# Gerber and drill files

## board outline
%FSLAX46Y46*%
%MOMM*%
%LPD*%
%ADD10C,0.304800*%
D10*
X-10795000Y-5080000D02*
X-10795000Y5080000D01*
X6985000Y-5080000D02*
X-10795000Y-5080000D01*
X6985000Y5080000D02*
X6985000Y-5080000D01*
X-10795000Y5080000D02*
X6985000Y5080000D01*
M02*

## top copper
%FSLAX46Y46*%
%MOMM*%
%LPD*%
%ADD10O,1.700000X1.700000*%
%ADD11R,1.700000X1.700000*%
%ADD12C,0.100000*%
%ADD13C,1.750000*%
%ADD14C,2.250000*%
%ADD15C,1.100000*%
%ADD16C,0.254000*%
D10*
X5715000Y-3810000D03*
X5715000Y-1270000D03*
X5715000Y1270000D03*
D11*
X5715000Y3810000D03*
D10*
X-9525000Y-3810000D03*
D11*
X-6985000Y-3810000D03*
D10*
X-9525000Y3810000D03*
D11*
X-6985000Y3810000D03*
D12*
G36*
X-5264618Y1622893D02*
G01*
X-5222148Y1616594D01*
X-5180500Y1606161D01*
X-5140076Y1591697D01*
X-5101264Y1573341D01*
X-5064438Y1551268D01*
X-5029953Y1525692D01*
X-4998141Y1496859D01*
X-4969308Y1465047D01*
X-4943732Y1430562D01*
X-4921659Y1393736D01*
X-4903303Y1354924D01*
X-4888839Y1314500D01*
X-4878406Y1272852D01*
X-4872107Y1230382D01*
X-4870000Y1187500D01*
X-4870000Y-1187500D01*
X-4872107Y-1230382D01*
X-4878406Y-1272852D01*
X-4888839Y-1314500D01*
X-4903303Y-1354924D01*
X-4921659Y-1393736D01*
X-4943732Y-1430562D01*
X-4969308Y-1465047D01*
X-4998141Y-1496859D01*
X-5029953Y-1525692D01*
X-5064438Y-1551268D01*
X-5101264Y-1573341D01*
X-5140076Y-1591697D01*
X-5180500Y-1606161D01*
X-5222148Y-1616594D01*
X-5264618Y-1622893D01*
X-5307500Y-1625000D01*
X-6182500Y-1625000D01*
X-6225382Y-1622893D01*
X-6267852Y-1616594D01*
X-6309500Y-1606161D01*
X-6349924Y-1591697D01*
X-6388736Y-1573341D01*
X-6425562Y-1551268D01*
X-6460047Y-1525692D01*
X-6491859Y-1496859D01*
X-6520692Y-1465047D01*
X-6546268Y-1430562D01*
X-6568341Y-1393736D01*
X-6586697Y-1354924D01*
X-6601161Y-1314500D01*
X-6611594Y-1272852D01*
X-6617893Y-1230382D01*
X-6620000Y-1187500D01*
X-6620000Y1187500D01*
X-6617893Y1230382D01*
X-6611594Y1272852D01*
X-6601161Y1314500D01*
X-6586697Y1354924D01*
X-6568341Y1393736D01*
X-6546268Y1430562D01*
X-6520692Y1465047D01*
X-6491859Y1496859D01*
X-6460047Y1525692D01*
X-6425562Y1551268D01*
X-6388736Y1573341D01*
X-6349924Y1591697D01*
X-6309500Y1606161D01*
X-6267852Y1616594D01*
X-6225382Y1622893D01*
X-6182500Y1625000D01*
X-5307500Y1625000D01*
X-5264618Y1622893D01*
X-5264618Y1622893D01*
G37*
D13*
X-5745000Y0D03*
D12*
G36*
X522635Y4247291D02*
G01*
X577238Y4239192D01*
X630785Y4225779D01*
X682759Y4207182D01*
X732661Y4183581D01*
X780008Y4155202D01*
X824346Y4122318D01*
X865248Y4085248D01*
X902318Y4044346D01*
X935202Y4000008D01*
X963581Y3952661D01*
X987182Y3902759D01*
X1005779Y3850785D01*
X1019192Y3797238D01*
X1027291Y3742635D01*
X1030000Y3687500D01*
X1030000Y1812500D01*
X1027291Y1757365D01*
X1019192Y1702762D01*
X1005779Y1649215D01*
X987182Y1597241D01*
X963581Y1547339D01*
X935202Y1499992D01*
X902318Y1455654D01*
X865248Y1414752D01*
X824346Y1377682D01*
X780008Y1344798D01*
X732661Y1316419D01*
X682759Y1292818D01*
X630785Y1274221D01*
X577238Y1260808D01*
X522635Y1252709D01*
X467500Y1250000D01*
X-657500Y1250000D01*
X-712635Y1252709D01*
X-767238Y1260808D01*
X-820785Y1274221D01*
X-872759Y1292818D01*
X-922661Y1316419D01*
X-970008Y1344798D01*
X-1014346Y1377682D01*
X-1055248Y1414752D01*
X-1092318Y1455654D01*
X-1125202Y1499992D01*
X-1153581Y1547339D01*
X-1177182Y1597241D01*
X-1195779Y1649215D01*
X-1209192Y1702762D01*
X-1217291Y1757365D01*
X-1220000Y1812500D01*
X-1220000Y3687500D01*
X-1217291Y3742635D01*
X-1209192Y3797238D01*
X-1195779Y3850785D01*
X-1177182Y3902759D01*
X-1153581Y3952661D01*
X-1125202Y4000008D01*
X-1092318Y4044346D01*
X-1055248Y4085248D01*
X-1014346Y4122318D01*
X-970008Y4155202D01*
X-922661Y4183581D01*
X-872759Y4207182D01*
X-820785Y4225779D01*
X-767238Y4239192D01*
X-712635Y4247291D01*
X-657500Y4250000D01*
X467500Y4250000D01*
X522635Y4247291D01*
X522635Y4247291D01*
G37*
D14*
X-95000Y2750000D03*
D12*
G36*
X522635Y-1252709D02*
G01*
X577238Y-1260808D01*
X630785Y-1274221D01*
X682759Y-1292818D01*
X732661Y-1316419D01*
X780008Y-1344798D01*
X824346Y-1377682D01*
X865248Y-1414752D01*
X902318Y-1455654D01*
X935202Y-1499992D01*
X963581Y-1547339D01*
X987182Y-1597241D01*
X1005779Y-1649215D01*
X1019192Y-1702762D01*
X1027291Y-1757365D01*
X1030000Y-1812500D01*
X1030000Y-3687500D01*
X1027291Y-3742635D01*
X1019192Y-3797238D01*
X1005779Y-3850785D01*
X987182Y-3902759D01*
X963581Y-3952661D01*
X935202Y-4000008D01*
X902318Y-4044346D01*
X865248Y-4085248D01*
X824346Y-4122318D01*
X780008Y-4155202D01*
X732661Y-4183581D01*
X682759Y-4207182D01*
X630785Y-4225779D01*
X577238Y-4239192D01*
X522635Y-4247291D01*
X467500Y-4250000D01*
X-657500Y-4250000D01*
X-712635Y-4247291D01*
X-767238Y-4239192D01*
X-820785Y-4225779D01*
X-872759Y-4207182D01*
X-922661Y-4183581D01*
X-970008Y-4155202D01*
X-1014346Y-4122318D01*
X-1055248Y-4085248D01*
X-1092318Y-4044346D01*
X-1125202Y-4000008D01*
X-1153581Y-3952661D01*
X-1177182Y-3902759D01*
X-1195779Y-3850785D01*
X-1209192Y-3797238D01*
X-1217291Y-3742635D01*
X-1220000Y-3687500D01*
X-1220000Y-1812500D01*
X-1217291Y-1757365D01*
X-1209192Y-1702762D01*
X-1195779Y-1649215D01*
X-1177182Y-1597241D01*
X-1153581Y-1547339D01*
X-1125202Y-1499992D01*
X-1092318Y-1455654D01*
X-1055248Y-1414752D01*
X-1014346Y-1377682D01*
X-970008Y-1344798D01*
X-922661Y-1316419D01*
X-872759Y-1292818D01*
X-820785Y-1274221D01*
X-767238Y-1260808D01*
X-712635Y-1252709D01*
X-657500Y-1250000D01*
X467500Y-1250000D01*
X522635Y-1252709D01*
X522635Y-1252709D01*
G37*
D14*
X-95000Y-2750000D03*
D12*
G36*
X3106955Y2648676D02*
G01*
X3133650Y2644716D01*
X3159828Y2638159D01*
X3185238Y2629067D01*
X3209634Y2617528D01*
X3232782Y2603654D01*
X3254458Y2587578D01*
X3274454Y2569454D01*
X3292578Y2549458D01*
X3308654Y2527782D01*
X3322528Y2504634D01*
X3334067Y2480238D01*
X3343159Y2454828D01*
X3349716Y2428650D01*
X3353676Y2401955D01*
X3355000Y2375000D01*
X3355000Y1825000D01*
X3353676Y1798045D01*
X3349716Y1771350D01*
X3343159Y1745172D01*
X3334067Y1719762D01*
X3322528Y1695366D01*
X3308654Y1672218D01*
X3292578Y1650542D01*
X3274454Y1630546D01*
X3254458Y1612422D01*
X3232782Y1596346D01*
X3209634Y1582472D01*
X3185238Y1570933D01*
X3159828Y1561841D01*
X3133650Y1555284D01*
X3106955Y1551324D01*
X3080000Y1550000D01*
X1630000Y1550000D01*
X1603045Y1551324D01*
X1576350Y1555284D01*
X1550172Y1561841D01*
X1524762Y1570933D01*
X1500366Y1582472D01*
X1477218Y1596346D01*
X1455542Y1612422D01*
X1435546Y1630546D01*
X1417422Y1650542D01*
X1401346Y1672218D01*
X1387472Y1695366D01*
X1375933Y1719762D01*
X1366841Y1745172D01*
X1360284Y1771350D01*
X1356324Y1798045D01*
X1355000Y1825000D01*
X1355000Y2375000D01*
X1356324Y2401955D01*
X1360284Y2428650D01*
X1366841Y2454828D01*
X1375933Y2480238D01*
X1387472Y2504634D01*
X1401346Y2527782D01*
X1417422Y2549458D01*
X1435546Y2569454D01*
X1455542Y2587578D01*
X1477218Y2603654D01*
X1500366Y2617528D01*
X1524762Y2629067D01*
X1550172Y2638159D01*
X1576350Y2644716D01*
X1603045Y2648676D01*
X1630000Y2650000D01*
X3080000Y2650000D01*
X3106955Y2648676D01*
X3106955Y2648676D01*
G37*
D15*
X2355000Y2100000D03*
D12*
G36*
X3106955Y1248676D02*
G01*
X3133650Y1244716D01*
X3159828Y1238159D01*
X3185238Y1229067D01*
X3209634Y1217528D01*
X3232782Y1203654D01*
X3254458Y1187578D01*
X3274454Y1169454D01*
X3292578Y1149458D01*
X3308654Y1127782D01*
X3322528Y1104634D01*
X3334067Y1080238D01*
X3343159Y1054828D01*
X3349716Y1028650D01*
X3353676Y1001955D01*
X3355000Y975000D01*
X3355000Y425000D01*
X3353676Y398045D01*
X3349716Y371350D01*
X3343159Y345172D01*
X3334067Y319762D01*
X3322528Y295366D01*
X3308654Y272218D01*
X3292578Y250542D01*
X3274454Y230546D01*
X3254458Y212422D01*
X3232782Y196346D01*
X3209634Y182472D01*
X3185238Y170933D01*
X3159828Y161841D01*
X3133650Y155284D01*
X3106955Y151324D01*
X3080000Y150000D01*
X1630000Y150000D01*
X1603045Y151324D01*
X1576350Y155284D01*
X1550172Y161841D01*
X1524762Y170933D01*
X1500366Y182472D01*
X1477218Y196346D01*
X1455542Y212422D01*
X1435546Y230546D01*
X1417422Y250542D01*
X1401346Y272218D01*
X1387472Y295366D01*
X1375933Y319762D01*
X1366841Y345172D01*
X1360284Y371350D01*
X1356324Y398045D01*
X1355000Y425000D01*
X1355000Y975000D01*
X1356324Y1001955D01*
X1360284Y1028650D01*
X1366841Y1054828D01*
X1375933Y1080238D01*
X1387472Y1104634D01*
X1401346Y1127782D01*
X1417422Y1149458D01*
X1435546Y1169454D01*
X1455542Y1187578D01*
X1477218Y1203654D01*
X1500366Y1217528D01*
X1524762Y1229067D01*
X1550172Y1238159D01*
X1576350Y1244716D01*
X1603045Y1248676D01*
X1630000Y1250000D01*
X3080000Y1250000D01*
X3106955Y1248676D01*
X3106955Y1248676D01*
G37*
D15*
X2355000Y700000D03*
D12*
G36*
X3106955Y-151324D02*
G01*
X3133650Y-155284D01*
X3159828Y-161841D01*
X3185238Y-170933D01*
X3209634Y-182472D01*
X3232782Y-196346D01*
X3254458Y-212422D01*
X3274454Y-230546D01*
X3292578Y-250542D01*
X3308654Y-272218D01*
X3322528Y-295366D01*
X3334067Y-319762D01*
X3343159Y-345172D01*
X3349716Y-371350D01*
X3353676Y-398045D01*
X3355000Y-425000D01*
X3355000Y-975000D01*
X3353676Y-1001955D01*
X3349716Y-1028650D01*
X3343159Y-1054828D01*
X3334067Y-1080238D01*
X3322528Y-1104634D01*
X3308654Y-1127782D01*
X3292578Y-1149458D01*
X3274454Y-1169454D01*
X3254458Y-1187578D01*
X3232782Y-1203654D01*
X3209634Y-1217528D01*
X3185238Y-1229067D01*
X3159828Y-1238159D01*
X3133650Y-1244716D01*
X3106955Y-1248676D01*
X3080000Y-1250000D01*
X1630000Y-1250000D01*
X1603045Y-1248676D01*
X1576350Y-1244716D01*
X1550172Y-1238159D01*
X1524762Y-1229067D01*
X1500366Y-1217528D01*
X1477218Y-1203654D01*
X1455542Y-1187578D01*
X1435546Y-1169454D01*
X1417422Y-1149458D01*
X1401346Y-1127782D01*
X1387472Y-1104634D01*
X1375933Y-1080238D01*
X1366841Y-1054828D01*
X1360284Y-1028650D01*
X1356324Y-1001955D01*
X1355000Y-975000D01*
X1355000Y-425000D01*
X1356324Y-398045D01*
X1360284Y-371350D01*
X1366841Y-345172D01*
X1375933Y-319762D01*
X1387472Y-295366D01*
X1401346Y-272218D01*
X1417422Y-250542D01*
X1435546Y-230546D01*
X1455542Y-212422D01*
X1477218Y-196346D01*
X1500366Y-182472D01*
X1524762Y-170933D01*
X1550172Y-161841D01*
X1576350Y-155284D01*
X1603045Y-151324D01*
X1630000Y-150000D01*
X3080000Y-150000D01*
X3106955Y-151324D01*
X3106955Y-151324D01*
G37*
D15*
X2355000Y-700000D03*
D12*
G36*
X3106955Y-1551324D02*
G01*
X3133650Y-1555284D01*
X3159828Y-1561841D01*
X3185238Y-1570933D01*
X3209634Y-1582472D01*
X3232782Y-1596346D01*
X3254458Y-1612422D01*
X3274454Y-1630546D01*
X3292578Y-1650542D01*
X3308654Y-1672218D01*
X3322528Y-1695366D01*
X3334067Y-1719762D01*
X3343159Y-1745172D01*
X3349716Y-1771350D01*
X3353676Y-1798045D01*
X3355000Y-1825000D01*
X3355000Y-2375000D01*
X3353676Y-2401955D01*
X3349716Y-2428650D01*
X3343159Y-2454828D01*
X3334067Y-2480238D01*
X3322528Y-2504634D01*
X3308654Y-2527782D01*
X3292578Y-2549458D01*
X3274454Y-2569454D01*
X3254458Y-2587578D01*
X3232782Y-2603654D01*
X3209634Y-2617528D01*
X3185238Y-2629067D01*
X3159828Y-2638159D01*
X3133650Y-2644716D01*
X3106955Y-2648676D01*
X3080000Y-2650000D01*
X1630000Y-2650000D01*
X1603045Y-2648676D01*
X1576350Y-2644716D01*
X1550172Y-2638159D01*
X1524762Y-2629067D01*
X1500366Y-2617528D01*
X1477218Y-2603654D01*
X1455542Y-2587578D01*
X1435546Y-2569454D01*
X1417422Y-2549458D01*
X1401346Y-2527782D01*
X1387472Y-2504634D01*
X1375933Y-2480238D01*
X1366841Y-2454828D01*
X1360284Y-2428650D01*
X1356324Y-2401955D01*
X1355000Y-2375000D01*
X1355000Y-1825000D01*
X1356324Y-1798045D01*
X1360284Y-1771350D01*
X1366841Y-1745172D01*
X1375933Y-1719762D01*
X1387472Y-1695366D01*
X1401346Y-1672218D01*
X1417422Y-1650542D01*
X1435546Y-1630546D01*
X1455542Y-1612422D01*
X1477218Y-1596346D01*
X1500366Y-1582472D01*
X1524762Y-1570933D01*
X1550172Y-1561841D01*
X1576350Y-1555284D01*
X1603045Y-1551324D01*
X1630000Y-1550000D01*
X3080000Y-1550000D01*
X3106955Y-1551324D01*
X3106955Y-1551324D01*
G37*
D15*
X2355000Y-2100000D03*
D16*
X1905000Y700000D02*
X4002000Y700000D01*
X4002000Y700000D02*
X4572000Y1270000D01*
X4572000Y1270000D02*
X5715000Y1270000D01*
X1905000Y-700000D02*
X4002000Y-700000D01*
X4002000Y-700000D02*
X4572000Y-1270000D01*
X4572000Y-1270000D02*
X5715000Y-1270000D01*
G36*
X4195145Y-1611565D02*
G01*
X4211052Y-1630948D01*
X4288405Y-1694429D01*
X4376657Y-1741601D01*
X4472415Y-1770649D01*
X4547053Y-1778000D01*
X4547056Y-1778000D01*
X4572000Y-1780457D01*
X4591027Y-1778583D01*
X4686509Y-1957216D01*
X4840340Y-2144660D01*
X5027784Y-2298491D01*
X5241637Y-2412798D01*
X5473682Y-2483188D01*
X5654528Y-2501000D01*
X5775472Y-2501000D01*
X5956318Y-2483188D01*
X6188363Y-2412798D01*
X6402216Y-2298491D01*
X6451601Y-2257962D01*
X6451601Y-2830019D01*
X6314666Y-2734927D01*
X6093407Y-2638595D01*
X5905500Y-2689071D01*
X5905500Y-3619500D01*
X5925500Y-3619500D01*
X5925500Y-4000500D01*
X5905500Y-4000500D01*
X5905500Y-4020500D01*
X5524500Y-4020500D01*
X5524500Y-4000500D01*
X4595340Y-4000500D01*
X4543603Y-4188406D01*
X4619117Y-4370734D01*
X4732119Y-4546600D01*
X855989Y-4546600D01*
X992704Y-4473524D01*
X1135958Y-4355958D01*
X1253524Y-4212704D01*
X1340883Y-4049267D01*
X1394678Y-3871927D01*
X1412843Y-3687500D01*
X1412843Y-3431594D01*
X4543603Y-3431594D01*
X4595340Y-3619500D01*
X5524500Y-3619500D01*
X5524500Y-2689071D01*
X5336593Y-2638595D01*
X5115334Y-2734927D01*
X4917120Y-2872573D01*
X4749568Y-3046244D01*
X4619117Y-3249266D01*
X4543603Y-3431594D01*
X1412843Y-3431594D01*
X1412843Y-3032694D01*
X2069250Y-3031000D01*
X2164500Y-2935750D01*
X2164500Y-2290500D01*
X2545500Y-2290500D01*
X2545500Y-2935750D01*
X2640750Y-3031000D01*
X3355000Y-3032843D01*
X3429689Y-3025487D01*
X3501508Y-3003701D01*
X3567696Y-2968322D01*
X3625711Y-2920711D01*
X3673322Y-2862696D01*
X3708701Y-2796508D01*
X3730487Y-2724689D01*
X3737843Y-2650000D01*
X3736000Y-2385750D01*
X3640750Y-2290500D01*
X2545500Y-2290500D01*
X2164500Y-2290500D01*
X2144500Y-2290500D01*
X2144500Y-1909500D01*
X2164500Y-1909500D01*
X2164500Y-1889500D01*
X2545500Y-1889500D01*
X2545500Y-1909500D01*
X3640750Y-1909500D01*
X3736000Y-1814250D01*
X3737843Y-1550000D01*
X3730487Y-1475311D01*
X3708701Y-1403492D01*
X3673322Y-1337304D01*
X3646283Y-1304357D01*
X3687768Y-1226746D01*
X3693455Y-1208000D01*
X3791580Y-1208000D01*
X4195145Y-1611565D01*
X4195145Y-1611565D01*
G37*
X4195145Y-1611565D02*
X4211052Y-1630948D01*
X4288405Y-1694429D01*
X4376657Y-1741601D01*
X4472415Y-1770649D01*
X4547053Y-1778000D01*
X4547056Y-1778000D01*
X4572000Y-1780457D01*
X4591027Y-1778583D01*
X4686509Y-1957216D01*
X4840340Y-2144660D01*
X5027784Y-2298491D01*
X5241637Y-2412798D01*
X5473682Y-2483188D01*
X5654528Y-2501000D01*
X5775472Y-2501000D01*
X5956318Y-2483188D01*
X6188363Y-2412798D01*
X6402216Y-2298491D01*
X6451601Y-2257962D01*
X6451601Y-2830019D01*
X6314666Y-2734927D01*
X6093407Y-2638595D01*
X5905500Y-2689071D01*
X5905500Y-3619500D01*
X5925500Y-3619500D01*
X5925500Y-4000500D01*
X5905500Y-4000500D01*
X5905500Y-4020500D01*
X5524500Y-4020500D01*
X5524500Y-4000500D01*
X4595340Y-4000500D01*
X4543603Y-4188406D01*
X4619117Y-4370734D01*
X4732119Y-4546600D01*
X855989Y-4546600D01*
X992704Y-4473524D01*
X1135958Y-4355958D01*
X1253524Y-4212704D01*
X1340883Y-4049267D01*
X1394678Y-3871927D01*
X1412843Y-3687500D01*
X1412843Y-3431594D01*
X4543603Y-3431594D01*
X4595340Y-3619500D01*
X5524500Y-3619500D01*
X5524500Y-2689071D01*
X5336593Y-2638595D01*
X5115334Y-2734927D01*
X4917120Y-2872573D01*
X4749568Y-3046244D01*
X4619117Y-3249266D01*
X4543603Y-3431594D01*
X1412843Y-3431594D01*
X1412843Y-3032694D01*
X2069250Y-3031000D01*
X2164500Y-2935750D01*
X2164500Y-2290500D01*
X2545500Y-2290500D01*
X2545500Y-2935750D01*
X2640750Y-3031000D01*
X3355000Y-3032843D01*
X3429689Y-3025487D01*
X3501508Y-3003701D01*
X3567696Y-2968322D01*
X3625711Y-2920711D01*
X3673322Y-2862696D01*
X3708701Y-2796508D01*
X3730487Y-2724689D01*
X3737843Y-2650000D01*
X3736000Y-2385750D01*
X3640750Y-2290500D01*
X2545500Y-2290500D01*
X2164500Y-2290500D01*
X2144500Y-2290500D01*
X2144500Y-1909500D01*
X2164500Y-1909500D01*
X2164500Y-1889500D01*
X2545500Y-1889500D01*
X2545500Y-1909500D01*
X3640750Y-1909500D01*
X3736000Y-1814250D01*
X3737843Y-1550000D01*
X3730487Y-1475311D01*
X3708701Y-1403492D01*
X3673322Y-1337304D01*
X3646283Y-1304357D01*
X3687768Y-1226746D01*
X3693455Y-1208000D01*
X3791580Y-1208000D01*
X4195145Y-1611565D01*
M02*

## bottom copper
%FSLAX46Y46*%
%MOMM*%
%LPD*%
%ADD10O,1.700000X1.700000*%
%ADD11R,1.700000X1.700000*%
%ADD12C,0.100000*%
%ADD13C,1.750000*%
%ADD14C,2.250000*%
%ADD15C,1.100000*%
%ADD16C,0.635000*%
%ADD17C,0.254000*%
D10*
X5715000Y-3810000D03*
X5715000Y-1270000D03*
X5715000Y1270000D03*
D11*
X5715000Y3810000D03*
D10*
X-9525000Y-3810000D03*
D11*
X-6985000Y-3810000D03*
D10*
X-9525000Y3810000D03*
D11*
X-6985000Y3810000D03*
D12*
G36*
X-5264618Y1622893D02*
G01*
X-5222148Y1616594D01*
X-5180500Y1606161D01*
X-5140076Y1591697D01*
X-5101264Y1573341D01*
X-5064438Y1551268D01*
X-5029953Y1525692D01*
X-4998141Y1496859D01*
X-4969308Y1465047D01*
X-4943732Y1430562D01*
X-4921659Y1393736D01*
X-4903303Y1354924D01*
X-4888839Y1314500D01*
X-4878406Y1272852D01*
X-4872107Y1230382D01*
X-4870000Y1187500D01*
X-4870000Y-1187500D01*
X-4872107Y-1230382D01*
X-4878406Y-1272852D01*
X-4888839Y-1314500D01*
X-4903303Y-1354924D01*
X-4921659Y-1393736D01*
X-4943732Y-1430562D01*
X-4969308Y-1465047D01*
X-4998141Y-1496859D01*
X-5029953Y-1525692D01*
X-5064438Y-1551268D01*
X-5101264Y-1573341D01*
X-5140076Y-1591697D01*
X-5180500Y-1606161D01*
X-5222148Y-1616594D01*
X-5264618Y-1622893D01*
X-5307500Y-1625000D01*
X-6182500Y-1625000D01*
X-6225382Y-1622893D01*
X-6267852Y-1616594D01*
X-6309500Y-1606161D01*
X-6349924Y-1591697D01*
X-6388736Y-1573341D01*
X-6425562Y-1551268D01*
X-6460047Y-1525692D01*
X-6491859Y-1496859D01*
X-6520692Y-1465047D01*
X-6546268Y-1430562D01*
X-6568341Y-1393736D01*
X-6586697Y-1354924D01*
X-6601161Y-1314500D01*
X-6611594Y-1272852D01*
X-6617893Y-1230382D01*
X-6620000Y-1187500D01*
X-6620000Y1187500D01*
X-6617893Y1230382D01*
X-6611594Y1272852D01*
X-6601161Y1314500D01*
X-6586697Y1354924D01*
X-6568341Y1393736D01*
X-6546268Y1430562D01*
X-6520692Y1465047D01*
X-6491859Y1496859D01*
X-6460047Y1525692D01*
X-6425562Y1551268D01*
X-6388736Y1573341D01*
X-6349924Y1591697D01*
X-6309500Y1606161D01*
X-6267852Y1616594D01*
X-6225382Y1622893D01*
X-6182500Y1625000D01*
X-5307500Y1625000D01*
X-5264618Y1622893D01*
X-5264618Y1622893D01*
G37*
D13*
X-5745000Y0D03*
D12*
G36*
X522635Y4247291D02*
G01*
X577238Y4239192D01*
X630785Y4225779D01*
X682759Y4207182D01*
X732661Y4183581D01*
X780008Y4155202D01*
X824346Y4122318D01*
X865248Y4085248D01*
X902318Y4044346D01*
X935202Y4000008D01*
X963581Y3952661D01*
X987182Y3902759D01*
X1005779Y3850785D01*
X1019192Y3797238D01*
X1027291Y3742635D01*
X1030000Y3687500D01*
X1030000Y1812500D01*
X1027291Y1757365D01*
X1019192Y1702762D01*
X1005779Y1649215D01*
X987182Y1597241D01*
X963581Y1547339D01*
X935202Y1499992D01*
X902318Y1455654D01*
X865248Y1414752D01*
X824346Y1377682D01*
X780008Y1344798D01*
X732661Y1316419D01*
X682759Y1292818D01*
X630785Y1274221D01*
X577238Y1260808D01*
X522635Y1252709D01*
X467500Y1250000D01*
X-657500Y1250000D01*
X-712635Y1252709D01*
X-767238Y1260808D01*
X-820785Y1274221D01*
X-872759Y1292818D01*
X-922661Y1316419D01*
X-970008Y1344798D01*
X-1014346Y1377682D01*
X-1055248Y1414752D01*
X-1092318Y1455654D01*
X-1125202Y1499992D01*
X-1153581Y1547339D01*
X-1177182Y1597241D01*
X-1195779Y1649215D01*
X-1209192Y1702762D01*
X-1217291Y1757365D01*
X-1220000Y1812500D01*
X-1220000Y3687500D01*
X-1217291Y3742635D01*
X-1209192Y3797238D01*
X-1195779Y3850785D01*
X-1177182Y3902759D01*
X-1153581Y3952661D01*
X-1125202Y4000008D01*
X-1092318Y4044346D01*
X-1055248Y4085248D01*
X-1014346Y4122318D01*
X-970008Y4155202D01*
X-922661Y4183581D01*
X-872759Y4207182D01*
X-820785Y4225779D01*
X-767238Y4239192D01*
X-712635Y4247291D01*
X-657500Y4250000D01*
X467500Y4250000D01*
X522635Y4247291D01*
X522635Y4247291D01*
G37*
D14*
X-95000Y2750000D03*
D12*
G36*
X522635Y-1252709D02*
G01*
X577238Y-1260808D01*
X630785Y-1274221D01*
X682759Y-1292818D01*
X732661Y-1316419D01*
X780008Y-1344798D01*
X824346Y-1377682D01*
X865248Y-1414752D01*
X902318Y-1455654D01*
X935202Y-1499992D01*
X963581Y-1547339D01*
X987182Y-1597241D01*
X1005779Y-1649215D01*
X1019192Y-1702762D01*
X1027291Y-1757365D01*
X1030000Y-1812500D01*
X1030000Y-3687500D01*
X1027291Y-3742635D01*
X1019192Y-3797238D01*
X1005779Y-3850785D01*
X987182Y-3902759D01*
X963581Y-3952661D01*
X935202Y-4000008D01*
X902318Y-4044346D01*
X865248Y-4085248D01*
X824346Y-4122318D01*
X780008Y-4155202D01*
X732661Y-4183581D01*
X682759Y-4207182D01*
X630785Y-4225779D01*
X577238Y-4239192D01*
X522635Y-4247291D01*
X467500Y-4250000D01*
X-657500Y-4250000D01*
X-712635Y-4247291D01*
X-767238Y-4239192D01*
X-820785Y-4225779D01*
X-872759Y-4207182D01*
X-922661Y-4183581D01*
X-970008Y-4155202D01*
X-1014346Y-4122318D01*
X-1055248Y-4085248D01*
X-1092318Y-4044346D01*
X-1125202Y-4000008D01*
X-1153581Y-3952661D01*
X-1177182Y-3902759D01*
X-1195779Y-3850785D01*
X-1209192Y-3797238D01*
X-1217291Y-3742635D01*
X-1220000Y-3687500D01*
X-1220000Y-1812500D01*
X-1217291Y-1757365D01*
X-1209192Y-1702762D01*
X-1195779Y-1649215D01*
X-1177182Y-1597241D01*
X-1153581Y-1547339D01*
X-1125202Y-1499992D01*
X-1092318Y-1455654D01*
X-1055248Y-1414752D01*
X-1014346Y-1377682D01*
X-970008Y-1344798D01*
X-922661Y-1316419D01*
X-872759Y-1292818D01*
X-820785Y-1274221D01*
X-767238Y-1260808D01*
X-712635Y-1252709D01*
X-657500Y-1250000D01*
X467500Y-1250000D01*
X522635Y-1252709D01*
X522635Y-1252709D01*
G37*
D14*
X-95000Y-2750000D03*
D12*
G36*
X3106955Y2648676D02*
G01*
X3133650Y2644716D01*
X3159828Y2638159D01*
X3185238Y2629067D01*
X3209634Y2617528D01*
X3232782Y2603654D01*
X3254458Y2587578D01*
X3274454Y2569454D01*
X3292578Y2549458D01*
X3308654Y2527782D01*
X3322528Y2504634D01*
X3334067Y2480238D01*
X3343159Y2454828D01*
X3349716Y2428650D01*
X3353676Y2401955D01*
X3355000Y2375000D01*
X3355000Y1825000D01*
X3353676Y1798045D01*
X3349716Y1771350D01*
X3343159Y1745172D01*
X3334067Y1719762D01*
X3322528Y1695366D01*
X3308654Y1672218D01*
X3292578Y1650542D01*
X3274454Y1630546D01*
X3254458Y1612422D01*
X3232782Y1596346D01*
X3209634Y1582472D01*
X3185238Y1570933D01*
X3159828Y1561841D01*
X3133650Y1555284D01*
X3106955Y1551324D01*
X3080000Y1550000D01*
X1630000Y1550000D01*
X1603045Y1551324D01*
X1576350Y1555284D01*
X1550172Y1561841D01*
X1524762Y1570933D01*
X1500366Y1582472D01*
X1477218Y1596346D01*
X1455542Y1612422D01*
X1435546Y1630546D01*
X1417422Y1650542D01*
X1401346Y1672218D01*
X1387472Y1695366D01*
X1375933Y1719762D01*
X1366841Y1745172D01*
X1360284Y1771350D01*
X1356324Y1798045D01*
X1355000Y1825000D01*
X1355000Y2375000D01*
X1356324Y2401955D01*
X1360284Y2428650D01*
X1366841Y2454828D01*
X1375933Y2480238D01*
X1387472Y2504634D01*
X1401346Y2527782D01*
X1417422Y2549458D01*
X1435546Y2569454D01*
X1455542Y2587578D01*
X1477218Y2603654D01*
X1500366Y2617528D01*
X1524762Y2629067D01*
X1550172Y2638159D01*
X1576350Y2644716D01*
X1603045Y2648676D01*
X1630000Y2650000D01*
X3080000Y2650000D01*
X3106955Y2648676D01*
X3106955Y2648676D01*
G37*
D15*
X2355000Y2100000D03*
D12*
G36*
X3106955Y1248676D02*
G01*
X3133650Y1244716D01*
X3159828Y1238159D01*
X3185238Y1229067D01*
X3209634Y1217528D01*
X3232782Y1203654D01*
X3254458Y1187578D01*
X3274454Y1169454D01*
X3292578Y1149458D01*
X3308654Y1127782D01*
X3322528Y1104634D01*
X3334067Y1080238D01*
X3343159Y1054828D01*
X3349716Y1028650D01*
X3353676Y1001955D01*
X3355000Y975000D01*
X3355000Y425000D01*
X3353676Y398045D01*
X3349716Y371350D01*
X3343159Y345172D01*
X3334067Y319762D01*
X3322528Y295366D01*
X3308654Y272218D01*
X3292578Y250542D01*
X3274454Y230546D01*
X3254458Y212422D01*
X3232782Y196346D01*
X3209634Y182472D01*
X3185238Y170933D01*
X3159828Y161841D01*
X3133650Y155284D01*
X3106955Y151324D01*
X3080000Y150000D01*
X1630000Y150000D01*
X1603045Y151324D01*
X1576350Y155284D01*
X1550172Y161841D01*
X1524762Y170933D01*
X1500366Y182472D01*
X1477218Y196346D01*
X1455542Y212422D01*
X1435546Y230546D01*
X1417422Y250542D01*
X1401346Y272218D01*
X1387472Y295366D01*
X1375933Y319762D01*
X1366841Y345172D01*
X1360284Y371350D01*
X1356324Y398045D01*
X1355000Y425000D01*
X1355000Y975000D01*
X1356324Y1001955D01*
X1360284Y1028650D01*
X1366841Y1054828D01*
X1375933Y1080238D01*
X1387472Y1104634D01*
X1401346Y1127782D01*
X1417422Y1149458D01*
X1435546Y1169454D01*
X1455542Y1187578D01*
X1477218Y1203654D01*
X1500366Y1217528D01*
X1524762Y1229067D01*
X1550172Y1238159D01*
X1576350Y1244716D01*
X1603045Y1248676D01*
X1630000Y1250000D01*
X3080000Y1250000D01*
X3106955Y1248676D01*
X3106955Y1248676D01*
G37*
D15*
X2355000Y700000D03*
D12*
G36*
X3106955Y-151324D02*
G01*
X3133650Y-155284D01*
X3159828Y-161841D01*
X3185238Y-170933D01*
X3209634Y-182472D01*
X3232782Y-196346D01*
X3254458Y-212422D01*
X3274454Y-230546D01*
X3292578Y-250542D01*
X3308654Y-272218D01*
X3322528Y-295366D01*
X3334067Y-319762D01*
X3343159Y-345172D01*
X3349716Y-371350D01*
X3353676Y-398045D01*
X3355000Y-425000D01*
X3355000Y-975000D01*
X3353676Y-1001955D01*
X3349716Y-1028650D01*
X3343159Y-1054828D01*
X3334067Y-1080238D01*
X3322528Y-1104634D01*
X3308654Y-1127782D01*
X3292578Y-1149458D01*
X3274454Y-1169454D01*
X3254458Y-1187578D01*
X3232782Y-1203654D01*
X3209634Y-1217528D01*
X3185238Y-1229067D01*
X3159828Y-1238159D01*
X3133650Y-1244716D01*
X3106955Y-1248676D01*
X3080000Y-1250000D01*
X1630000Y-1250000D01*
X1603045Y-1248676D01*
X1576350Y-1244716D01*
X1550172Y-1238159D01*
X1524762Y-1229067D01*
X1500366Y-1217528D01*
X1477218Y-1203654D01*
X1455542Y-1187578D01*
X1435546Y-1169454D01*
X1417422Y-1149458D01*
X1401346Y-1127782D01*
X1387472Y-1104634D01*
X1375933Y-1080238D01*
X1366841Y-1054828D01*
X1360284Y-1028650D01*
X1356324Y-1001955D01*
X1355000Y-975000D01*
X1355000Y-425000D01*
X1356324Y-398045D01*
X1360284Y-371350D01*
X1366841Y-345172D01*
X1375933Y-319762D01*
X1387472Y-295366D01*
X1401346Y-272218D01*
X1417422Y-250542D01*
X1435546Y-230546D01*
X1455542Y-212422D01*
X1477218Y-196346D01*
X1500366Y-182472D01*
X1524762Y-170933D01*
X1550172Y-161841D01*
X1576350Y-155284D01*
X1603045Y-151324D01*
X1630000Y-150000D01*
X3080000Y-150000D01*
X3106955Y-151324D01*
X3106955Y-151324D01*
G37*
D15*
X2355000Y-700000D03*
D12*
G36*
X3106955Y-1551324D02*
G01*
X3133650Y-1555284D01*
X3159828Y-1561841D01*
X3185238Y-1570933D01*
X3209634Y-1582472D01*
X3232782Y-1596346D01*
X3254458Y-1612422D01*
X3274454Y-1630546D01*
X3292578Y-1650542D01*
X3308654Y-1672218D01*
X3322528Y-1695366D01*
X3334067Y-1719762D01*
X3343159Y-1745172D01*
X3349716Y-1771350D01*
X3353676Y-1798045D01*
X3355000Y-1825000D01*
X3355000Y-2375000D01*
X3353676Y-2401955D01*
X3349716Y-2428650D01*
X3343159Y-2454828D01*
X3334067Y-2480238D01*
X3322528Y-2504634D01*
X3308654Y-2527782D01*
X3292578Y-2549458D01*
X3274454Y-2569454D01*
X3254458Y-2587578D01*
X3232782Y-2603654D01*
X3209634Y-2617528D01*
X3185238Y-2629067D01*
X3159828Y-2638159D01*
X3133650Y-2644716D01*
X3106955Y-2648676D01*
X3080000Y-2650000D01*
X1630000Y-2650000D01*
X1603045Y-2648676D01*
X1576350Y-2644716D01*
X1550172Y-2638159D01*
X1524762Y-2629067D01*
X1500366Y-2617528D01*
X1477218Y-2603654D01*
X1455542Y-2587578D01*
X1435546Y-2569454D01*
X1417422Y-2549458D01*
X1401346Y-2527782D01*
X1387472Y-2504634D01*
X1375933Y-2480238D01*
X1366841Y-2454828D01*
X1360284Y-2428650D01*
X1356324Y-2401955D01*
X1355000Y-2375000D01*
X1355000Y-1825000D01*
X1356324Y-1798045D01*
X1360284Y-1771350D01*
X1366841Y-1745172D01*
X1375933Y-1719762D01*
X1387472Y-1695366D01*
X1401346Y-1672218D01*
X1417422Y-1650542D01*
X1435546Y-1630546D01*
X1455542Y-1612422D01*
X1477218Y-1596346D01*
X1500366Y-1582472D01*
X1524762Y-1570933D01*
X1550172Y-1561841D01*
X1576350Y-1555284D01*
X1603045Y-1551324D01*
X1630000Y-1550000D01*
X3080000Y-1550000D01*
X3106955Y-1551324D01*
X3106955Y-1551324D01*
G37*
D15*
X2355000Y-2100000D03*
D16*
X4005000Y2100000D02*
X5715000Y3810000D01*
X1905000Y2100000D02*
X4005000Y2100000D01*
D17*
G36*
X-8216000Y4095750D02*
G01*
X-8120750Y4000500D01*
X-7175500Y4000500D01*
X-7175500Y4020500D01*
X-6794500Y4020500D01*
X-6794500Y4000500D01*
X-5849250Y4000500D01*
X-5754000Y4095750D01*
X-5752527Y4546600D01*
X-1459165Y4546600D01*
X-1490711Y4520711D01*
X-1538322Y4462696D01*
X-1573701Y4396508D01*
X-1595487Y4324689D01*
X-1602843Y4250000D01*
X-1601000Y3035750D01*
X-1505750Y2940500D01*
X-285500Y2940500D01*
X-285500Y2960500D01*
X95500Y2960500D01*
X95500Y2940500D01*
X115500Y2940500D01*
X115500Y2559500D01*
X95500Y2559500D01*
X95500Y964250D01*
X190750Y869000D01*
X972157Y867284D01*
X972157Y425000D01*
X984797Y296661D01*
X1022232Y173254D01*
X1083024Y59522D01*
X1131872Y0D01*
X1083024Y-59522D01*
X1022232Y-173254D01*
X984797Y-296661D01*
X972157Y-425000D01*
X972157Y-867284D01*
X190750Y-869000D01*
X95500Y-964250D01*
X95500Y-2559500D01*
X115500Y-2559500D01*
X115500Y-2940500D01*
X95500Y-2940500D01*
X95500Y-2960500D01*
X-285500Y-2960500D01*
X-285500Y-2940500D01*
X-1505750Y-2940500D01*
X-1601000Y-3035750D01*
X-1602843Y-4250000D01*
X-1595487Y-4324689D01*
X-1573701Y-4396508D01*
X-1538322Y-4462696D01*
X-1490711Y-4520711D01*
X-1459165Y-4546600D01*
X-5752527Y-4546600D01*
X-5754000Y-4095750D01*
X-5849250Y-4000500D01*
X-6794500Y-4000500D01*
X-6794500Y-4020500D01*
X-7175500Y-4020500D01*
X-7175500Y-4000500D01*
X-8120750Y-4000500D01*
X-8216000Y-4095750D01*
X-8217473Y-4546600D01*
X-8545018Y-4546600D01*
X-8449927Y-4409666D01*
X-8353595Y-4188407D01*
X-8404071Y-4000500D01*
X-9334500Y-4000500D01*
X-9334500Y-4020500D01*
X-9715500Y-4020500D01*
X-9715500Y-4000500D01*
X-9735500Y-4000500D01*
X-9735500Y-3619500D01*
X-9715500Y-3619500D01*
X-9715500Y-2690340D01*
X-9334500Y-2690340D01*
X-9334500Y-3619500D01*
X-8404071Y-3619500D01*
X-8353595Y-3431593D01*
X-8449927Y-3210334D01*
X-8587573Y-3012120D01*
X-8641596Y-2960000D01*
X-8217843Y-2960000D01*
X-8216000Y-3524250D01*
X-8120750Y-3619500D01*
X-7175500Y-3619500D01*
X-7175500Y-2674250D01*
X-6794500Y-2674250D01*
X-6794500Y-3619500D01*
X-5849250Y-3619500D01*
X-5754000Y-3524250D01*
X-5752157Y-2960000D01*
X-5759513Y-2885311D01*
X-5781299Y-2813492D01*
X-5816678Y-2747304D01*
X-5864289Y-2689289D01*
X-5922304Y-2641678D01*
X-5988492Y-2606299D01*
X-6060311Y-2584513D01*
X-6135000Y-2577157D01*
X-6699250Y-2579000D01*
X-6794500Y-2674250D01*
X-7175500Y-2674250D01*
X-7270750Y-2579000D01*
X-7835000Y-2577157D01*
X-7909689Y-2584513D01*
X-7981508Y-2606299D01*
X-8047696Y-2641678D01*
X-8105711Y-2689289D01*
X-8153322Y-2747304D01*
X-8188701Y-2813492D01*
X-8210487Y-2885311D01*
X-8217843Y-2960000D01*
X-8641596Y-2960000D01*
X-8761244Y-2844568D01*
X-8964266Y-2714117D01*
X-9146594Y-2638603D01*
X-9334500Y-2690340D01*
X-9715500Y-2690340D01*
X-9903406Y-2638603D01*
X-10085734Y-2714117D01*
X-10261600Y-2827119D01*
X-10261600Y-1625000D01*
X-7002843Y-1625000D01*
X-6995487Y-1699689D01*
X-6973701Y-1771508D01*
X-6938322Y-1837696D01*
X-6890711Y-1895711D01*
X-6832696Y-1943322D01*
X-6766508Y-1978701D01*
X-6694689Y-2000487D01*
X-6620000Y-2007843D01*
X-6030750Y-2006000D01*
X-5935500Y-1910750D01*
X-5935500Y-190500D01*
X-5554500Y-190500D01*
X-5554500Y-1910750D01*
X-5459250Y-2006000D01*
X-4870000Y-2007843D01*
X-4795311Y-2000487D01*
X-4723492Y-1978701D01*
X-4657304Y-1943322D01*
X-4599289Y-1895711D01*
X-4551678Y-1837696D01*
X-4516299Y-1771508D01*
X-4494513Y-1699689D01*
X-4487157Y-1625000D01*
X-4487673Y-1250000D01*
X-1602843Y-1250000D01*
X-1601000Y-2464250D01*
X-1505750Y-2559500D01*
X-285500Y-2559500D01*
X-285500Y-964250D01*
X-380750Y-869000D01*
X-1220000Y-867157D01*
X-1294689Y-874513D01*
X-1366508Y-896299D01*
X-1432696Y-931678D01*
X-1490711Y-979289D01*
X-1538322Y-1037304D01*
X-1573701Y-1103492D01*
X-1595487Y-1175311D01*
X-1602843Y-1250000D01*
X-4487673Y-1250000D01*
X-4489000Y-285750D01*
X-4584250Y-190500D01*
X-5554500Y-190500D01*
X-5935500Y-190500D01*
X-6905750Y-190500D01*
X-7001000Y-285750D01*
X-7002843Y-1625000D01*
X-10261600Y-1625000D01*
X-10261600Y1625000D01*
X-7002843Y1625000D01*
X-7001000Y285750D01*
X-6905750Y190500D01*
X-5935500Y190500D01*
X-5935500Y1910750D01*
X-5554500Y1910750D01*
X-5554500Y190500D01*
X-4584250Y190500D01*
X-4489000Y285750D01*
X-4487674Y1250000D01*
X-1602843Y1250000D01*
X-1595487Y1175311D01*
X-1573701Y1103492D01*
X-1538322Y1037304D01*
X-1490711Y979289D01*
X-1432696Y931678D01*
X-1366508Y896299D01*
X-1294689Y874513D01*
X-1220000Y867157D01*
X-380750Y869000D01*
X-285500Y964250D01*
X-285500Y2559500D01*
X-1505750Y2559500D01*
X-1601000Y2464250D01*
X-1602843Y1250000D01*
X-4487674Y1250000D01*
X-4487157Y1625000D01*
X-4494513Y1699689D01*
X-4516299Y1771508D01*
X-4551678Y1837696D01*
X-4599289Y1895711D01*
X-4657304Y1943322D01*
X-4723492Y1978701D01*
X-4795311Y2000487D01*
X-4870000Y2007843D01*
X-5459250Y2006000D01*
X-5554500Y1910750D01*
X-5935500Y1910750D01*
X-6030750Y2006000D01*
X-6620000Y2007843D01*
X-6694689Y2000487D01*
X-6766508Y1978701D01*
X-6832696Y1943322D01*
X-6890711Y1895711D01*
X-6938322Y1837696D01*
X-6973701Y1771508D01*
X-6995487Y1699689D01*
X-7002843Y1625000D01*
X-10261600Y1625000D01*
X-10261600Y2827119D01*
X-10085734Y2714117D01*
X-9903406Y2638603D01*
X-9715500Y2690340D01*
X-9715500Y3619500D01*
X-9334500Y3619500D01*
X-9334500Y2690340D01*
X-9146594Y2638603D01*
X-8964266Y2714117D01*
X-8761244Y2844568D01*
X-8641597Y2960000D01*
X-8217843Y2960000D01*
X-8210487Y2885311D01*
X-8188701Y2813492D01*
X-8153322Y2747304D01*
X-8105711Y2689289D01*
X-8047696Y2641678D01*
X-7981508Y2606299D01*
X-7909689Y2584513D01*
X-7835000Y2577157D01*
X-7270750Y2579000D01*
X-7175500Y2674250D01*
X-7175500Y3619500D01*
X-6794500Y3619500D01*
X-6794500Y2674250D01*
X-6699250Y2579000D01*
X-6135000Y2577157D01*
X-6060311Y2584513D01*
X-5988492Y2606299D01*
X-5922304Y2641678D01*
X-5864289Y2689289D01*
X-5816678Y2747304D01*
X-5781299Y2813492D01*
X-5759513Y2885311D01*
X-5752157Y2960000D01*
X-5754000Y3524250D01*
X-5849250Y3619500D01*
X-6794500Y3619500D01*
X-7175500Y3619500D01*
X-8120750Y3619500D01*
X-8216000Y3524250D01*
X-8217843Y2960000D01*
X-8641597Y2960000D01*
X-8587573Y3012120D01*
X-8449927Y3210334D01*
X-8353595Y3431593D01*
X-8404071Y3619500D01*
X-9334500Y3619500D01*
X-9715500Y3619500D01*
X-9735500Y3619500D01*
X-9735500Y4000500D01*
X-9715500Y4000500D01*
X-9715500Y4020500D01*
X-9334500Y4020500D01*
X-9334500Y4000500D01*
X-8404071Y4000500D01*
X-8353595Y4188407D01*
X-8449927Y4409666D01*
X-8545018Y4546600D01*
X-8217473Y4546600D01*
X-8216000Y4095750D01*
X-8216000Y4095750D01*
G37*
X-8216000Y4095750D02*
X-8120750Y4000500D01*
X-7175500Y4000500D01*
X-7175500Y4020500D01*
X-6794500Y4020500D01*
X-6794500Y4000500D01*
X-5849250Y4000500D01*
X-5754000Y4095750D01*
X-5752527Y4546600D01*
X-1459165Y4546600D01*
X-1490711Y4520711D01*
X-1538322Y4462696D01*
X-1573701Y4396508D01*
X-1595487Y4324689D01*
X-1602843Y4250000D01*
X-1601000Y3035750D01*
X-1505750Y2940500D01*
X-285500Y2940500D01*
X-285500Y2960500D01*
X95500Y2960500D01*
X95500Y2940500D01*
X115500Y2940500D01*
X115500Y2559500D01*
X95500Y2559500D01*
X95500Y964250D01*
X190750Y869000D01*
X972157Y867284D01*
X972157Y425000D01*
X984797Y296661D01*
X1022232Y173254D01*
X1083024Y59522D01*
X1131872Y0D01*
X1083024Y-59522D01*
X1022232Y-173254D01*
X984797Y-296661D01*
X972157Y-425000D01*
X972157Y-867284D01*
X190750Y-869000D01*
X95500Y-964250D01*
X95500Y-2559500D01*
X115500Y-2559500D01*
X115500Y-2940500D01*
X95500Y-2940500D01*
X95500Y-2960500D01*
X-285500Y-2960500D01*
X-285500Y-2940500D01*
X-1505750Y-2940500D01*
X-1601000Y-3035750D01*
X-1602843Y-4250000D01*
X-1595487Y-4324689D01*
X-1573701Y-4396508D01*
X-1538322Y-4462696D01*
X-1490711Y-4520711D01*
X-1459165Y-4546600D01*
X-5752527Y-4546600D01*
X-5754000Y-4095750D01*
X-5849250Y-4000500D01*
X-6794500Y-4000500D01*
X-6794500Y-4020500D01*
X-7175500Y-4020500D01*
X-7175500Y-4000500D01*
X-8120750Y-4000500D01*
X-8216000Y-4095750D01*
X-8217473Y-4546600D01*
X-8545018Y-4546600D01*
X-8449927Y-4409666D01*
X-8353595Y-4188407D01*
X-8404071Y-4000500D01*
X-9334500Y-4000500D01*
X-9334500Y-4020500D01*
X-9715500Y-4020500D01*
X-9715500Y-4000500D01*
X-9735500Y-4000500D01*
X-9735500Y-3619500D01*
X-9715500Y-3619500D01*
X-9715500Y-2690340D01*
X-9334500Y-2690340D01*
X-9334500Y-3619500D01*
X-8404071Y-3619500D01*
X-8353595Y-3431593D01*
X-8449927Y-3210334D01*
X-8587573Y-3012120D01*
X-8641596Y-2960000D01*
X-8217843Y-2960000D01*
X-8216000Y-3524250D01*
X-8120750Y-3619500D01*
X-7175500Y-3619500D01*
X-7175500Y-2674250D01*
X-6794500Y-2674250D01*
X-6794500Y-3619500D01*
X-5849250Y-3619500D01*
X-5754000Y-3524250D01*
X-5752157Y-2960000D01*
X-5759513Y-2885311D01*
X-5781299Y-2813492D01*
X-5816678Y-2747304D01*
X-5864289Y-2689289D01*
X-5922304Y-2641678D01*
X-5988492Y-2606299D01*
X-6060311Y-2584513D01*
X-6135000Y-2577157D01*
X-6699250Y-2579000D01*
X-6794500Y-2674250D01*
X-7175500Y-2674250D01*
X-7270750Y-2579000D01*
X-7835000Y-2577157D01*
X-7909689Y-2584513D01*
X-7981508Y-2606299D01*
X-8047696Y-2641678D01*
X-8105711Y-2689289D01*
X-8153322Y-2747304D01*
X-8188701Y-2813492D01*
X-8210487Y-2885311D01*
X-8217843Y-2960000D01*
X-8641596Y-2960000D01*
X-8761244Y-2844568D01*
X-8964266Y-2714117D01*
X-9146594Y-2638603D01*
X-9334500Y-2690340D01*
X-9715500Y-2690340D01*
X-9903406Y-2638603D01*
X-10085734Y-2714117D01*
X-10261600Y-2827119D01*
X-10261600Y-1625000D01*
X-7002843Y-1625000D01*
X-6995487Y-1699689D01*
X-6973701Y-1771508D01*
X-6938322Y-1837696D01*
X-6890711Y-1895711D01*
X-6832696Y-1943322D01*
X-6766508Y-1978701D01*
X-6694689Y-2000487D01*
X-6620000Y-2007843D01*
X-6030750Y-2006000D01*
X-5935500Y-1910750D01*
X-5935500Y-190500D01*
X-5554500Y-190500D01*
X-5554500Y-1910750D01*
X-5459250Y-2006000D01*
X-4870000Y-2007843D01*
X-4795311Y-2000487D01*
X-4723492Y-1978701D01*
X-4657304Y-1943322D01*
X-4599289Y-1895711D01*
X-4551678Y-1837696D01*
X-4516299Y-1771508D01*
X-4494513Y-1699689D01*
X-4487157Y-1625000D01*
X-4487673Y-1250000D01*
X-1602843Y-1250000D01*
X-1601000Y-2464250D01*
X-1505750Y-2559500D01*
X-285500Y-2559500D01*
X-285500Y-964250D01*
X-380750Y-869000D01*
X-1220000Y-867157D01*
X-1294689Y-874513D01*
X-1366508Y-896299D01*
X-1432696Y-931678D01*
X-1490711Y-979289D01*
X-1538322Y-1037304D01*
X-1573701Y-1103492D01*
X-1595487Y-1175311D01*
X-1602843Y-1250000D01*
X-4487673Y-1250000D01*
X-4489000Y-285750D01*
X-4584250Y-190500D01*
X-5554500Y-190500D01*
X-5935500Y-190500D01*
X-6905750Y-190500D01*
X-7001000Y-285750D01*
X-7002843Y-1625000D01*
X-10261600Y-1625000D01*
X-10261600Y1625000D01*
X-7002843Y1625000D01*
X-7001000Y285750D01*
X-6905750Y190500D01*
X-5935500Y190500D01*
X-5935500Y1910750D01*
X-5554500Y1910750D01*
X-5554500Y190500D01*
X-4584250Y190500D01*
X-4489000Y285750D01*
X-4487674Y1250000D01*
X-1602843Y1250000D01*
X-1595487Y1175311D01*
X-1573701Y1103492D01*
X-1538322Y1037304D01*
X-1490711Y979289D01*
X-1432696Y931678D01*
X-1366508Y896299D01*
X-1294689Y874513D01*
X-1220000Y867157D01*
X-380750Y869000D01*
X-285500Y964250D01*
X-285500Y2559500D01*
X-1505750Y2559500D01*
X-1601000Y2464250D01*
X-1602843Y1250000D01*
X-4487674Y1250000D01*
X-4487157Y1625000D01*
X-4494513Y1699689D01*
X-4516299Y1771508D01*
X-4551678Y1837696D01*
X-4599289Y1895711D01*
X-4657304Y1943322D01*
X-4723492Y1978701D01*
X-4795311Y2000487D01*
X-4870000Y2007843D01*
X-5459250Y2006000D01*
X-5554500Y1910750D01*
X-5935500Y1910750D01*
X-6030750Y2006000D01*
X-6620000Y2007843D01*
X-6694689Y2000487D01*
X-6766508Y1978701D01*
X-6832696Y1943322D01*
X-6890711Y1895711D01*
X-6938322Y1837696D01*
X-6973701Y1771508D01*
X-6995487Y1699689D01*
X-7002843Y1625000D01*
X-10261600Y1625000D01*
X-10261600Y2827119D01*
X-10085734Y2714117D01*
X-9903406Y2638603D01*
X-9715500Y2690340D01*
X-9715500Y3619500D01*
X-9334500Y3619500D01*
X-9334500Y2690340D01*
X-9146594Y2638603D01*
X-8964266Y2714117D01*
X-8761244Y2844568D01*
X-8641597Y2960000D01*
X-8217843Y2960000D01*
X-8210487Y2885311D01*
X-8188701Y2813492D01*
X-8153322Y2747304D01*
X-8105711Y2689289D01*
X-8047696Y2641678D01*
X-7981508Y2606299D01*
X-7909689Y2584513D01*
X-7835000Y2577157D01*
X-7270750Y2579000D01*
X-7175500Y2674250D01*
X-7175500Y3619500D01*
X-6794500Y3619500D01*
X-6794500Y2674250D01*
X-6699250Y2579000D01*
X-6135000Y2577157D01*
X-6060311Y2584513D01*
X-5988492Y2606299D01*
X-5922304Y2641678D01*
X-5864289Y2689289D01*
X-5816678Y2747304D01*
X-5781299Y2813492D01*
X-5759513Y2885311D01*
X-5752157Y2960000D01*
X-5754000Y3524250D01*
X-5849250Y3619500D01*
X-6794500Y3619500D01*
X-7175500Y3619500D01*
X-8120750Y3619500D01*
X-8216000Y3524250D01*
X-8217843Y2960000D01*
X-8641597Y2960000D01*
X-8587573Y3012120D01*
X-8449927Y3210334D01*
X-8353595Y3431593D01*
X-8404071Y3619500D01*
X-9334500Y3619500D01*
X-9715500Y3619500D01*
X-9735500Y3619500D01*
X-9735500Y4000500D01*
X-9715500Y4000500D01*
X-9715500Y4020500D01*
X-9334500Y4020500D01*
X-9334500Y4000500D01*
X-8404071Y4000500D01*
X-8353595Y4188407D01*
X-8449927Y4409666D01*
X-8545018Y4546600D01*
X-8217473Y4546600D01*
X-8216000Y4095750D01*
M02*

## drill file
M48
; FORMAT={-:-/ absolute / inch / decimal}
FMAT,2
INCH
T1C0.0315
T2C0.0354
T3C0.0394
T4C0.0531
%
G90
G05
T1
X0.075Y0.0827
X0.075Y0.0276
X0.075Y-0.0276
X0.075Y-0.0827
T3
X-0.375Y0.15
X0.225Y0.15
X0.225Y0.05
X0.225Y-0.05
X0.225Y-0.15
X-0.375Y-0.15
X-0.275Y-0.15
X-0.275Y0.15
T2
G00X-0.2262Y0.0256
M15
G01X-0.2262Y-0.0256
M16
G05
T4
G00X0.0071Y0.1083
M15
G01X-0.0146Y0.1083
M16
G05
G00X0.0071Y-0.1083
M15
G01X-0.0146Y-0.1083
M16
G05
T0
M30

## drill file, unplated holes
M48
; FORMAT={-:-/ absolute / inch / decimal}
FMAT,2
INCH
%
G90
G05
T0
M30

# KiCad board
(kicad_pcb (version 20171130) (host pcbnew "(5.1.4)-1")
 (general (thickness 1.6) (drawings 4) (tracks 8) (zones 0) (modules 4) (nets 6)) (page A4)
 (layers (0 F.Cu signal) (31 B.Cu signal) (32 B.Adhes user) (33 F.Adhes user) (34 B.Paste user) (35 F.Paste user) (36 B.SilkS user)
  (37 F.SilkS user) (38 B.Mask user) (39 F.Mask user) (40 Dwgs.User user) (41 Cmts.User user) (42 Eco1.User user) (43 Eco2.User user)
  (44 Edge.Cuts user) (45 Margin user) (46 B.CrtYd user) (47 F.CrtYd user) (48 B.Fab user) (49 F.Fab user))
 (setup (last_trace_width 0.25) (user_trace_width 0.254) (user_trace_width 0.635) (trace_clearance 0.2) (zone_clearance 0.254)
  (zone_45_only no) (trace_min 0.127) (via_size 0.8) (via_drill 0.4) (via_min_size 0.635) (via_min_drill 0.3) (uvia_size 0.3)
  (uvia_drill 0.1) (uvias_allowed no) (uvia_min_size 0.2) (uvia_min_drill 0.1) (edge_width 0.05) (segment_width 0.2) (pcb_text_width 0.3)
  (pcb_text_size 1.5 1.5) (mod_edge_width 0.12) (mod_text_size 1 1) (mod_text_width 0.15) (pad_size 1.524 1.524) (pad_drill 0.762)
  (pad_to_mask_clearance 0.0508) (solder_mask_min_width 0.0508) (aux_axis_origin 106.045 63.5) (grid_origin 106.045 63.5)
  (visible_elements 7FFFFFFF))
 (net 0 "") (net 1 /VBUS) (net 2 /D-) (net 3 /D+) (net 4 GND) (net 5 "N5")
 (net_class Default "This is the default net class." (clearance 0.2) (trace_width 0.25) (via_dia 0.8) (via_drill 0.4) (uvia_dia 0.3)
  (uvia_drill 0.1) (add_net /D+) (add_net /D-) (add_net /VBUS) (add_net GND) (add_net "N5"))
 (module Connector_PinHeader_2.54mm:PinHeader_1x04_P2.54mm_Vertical (layer B.Cu) (at 111.76 59.69 180)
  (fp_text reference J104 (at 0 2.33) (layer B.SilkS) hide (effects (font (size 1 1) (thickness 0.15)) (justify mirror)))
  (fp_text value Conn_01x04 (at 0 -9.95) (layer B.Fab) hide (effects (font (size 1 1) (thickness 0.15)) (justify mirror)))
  (pad 4 thru_hole oval (at 0 -7.62 180) (size 1.7 1.7) (drill 1) (layers *.Cu *.Mask) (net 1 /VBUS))
  (pad 3 thru_hole oval (at 0 -5.08 180) (size 1.7 1.7) (drill 1) (layers *.Cu *.Mask) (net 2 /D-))
  (pad 2 thru_hole oval (at 0 -2.54 180) (size 1.7 1.7) (drill 1) (layers *.Cu *.Mask) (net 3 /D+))
  (pad 1 thru_hole rect (at 0 0 180) (size 1.7 1.7) (drill 1) (layers *.Cu *.Mask) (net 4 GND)))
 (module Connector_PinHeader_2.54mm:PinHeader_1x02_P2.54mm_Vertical (layer B.Cu) (at 99.06 67.31 90)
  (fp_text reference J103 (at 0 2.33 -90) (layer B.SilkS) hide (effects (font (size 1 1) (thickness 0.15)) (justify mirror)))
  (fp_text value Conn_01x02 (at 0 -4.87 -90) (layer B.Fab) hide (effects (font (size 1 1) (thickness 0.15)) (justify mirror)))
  (pad 2 thru_hole oval (at 0 -2.54 90) (size 1.7 1.7) (drill 1) (layers *.Cu *.Mask) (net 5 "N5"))
  (pad 1 thru_hole rect (at 0 0 90) (size 1.7 1.7) (drill 1) (layers *.Cu *.Mask) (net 5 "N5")))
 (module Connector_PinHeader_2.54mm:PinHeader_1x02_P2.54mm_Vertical (layer B.Cu) (at 99.06 59.69 90)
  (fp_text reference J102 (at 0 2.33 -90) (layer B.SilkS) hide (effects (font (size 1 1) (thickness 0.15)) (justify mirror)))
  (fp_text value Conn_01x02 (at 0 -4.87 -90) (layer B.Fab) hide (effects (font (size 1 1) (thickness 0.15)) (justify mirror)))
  (pad 2 thru_hole oval (at 0 -2.54 90) (size 1.7 1.7) (drill 1) (layers *.Cu *.Mask) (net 5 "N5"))
  (pad 1 thru_hole rect (at 0 0 90) (size 1.7 1.7) (drill 1) (layers *.Cu *.Mask) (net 5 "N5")))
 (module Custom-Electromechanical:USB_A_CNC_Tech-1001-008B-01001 (layer F.Cu) (at 107.95 63.5 270)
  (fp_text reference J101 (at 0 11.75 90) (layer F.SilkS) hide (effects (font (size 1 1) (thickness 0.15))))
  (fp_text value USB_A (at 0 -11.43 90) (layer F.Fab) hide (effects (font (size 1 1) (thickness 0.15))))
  (pad 5 thru_hole roundrect (at 0 7.65 270) (size 3.25 1.75) (drill oval 2.2 0.9) (layers *.Cu *.Mask) (roundrect_rratio 0.25) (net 5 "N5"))
  (pad 5 thru_hole roundrect (at -2.75 2 270) (size 3 2.25) (drill oval 1.35 1.9) (layers *.Cu *.Mask) (roundrect_rratio 0.25) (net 5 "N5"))
  (pad 5 thru_hole roundrect (at 2.75 2 270) (size 3 2.25) (drill oval 1.35 1.9) (layers *.Cu *.Mask) (roundrect_rratio 0.25) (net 5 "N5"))
  (pad 4 thru_hole roundrect (at -2.1 0 270) (size 1.1 2) (drill 0.8 (offset 0 -0.45)) (layers *.Cu *.Mask) (roundrect_rratio 0.25)
   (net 4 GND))
  (pad 3 thru_hole roundrect (at -0.7 0 270) (size 1.1 2) (drill 0.8 (offset 0 -0.45)) (layers *.Cu *.Mask) (roundrect_rratio 0.25)
   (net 3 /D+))
  (pad 2 thru_hole roundrect (at 0.7 0 270) (size 1.1 2) (drill 0.8 (offset 0 -0.45)) (layers *.Cu *.Mask) (roundrect_rratio 0.25)
   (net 2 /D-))
  (pad 1 thru_hole roundrect (at 2.1 0 270) (size 1.1 2) (drill 0.8 (offset 0 -0.45)) (layers *.Cu *.Mask) (roundrect_rratio 0.25)
   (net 1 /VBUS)))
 (gr_line (start 95.25 68.58) (end 95.25 58.42) (layer Edge.Cuts) (width 0.3048))
 (gr_line (start 113.03 68.58) (end 95.25 68.58) (layer Edge.Cuts) (width 0.3048))
 (gr_line (start 113.03 58.42) (end 113.03 68.58) (layer Edge.Cuts) (width 0.3048))
 (gr_line (start 95.25 58.42) (end 113.03 58.42) (layer Edge.Cuts) (width 0.3048))
 (segment (start 110.05 61.4) (end 111.76 59.69) (width 0.635) (layer B.Cu) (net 4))
 (segment (start 107.95 61.4) (end 110.05 61.4) (width 0.635) (layer B.Cu) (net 4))
 (segment (start 107.95 62.8) (end 110.047 62.8) (width 0.254) (layer F.Cu) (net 3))
 (segment (start 110.047 62.8) (end 110.617 62.23) (width 0.254) (layer F.Cu) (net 3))
 (segment (start 110.617 62.23) (end 111.76 62.23) (width 0.254) (layer F.Cu) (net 3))
 (segment (start 107.95 64.2) (end 110.047 64.2) (width 0.254) (layer F.Cu) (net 2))
 (segment (start 110.047 64.2) (end 110.617 64.77) (width 0.254) (layer F.Cu) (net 2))
 (segment (start 110.617 64.77) (end 111.76 64.77) (width 0.254) (layer F.Cu) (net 2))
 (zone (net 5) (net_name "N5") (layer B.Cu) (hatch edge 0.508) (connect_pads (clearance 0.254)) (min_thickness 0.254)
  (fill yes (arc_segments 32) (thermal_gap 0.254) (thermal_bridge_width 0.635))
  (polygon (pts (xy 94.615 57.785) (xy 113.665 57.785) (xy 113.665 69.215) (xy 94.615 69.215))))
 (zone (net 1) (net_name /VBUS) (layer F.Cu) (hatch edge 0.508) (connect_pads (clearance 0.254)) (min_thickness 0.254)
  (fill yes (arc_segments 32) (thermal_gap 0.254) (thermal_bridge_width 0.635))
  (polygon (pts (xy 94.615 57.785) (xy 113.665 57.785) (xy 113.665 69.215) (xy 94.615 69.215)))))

